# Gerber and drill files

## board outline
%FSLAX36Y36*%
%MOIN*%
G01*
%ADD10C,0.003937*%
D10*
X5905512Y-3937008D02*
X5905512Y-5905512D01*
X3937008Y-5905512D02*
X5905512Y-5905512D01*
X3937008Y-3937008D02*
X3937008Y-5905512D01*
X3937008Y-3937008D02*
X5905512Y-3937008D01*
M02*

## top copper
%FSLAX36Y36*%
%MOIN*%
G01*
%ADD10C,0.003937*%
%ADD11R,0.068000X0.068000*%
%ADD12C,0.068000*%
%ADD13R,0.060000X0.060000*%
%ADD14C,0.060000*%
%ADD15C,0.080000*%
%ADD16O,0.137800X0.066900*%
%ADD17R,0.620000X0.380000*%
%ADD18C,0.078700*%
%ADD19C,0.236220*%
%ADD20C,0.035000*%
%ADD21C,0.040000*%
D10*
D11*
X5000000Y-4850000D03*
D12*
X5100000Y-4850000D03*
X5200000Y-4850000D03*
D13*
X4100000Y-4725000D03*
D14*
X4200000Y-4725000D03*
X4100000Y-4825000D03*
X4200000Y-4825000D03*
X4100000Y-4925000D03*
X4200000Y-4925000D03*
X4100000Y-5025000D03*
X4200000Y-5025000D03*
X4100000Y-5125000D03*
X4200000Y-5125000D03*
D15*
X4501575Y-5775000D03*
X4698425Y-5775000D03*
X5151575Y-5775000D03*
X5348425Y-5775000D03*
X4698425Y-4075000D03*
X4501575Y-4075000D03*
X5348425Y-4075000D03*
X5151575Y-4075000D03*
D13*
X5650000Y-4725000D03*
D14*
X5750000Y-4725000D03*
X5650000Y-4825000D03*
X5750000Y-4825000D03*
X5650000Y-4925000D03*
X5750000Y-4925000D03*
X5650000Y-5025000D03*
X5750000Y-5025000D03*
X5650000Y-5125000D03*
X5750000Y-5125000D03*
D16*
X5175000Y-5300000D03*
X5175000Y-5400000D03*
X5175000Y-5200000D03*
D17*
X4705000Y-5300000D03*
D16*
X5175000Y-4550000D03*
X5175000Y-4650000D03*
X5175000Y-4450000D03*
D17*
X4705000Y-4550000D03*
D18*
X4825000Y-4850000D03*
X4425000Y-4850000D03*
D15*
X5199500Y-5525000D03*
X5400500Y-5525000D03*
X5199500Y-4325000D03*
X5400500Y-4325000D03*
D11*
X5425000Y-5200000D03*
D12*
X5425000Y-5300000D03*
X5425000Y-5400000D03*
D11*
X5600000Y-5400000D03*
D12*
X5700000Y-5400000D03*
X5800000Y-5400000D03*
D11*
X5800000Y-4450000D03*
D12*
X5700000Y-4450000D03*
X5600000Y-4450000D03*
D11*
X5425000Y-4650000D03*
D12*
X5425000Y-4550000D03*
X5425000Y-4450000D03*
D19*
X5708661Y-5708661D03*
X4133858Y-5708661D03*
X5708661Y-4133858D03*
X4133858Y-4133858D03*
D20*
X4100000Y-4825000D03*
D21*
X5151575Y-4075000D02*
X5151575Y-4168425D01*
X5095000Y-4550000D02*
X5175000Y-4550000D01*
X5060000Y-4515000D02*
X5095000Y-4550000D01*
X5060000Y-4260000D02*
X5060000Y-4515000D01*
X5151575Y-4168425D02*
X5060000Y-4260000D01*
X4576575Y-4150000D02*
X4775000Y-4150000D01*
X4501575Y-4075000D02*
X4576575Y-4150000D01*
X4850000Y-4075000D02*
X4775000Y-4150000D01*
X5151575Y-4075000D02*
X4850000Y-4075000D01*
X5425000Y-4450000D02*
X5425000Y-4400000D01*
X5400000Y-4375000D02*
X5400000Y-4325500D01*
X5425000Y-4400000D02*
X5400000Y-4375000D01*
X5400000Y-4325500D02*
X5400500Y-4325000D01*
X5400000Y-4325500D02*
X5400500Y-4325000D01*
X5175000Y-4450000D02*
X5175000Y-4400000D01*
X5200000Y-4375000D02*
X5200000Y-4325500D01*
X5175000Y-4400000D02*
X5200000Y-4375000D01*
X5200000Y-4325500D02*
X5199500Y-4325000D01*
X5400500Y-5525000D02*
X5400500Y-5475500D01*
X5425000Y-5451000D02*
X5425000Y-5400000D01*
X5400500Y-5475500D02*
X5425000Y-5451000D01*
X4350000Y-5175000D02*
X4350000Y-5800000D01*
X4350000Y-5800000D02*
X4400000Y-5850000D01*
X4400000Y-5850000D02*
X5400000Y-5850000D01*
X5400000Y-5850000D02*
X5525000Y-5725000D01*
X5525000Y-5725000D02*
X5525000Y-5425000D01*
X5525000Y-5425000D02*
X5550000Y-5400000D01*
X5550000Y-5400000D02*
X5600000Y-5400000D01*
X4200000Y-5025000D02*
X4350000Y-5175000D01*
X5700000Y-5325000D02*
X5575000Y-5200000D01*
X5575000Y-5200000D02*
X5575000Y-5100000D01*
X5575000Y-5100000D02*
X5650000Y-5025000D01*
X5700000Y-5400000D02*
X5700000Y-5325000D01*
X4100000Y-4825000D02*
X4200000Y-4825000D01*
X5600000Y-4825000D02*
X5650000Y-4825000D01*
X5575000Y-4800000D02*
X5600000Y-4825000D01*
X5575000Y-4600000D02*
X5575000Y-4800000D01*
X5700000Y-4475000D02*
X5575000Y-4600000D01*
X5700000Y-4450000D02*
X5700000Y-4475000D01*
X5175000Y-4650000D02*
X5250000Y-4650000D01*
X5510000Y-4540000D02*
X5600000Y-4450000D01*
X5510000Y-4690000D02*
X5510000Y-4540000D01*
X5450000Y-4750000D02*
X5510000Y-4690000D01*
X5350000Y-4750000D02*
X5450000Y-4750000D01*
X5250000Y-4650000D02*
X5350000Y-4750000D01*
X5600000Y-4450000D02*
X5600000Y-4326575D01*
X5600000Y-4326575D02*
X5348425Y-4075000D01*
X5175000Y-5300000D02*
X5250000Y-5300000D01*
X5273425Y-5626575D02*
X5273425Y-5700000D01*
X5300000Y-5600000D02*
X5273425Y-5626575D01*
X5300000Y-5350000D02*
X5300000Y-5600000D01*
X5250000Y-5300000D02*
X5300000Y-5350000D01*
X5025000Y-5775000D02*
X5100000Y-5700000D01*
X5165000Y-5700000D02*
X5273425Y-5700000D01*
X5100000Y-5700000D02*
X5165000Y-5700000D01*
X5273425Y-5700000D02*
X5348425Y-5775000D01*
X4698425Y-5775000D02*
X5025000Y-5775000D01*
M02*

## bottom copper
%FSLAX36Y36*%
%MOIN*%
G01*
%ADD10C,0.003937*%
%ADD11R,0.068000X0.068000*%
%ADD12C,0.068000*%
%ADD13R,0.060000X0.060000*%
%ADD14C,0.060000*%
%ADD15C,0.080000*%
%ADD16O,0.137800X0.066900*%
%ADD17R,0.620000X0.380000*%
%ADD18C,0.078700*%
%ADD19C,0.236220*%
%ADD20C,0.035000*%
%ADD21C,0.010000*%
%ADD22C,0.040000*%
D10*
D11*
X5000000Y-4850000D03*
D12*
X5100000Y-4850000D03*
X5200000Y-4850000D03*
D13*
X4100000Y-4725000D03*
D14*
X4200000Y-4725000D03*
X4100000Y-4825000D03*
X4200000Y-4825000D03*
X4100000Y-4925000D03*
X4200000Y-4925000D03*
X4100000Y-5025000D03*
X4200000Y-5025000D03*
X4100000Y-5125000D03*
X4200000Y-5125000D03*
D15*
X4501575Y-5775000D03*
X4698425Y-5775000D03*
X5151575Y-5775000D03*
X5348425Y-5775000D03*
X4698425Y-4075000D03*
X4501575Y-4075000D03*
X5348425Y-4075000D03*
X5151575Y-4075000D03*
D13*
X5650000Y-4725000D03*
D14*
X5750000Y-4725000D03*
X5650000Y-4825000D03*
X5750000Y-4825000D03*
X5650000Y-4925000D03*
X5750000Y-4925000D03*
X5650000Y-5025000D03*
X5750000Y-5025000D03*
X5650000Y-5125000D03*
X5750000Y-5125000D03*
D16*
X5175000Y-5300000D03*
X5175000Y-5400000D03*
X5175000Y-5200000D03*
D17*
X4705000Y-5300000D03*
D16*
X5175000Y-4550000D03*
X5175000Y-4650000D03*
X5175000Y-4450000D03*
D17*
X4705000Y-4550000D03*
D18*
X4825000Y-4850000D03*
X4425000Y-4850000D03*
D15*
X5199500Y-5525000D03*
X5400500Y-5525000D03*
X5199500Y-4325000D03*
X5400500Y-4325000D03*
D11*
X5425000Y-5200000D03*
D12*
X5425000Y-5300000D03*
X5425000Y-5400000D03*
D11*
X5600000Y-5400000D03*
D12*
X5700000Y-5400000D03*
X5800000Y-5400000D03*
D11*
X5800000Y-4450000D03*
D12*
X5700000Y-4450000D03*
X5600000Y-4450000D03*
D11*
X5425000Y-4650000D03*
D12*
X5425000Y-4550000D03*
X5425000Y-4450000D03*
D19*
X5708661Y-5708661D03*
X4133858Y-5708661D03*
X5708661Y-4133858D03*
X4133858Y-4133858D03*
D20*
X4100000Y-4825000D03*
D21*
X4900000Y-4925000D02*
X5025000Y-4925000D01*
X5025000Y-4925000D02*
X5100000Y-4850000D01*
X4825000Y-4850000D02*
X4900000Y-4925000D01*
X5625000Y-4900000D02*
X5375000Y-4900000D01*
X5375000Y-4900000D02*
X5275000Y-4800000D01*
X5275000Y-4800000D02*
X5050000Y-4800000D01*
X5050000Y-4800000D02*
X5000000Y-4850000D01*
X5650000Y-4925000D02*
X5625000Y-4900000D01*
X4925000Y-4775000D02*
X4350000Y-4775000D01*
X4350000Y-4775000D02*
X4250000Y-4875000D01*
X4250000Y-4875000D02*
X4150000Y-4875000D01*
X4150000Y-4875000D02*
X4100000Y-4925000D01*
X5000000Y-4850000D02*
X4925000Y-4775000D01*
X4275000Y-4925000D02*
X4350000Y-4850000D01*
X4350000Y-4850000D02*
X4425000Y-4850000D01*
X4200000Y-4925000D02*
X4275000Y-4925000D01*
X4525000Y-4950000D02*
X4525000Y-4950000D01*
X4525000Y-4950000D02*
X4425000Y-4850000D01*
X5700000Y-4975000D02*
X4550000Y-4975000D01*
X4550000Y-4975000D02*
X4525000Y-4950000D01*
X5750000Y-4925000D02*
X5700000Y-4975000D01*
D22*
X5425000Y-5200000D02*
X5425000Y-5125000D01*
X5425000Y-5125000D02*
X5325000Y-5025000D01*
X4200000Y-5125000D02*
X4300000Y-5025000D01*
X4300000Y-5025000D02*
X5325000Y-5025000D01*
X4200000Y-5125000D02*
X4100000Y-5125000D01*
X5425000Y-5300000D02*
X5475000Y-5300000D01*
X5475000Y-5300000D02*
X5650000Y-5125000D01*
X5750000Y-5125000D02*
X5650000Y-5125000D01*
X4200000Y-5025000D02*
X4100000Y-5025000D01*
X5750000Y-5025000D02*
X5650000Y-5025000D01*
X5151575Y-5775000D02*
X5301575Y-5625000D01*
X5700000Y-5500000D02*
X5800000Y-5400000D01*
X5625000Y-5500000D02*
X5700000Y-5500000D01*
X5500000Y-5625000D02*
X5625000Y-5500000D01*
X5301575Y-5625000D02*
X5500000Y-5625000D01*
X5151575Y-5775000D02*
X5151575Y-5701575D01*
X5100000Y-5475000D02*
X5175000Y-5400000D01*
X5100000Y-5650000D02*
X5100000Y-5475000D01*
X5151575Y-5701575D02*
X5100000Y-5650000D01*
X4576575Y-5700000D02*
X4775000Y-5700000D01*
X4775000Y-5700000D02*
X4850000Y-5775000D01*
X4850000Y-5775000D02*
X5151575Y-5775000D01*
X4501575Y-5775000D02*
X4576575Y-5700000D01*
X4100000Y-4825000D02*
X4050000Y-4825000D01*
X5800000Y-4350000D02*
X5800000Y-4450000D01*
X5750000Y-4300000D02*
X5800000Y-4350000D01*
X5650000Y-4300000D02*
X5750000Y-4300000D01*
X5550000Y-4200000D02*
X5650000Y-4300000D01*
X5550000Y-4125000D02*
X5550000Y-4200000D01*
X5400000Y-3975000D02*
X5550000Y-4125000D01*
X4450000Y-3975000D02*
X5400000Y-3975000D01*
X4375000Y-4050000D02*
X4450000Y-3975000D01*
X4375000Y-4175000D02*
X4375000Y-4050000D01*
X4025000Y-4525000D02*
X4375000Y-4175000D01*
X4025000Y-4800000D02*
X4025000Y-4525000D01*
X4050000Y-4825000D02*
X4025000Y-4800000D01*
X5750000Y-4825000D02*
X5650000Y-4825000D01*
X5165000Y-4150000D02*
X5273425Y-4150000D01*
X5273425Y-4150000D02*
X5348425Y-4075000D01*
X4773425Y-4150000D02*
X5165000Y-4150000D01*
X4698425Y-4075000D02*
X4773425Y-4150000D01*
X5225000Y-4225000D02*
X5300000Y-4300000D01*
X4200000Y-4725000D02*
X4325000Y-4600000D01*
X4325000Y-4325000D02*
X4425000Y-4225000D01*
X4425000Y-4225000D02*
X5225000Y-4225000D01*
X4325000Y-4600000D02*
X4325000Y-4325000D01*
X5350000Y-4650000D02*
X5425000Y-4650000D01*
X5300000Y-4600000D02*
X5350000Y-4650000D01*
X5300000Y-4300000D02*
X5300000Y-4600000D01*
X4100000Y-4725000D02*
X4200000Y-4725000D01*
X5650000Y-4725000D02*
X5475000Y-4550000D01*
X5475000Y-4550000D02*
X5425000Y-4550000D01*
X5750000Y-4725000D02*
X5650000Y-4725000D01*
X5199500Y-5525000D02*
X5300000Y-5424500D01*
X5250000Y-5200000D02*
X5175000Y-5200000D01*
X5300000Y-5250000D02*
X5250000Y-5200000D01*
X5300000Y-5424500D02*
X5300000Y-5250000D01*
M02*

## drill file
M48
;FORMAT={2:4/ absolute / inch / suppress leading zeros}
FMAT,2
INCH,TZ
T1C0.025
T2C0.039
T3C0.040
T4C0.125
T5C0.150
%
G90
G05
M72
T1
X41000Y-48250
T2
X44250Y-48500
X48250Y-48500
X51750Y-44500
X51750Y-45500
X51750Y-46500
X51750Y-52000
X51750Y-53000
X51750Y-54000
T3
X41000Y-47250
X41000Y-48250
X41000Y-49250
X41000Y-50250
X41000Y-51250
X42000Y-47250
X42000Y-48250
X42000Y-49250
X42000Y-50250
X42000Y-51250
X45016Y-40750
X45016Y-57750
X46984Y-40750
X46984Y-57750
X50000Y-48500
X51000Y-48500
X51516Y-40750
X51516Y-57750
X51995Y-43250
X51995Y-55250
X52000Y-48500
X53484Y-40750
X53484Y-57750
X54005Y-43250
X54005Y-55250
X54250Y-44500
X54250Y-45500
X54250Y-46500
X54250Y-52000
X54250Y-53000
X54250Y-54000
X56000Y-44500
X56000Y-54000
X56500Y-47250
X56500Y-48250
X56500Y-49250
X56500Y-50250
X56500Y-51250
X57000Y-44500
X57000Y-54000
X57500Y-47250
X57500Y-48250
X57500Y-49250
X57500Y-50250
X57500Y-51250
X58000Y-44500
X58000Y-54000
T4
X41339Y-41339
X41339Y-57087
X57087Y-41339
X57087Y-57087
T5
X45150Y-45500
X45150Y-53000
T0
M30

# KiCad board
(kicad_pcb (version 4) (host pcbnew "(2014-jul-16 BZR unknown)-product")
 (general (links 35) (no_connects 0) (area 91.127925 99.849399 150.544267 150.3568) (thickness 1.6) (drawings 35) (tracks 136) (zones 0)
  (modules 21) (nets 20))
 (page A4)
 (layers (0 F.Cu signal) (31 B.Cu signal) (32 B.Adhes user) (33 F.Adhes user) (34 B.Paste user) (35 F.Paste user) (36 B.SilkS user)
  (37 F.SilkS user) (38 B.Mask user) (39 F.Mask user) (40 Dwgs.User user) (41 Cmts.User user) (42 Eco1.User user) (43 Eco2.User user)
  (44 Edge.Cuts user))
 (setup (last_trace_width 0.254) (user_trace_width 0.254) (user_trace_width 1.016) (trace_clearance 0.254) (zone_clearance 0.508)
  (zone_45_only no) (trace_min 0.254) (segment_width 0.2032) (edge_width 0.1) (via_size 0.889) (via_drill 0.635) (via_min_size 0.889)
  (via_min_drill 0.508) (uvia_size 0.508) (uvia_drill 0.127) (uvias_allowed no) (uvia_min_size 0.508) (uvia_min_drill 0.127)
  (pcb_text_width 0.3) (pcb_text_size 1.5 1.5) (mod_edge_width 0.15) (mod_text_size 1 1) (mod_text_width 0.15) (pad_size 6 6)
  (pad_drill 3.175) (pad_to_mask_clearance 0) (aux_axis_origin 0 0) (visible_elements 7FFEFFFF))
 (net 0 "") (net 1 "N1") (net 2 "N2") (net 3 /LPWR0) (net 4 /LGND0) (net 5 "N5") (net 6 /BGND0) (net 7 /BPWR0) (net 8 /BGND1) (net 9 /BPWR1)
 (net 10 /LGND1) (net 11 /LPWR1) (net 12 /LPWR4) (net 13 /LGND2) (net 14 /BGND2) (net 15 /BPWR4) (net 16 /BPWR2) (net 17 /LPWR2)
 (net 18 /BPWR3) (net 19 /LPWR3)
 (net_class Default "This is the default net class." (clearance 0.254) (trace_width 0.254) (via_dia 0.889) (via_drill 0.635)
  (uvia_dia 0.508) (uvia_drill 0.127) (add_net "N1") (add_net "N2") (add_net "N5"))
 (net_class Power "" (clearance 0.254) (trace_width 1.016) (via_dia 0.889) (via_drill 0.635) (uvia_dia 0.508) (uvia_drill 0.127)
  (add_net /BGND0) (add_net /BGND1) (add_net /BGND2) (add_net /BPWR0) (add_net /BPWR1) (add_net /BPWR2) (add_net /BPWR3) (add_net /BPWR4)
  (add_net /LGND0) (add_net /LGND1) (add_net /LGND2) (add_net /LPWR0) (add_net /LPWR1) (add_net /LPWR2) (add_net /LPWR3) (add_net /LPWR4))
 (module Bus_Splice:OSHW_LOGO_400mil (layer B.Cu) (at 124.333 113.03 180)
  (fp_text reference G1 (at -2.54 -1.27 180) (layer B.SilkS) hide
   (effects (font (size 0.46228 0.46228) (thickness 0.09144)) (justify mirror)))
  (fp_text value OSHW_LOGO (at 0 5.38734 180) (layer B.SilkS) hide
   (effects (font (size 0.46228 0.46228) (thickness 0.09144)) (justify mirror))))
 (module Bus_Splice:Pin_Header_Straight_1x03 (layer F.Cu) (at 129.54 123.19)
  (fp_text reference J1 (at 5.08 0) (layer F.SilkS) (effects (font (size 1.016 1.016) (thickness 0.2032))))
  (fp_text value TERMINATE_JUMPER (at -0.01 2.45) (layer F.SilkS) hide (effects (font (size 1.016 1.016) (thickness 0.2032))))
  (pad 1 thru_hole rect (at -2.54 0) (size 1.7272 1.7272) (drill 1.016) (layers *.Cu *.Mask F.SilkS) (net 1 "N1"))
  (pad 2 thru_hole circle (at 0 0) (size 1.7272 1.7272) (drill 1.016) (layers *.Cu *.Mask F.SilkS) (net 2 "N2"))
  (pad 3 thru_hole circle (at 2.54 0) (size 1.7272 1.7272) (drill 1.016) (layers *.Cu *.Mask F.SilkS)))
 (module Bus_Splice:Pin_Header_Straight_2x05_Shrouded (layer F.Cu) (at 105.41 125.095 270)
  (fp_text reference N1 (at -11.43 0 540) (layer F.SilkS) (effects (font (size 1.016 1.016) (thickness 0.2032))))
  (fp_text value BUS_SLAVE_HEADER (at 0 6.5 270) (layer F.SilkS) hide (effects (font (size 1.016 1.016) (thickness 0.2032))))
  (pad 1 thru_hole rect (at -5.08 1.27 270) (size 1.524 1.524) (drill 1.016) (layers *.Cu *.Mask F.SilkS) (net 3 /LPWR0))
  (pad 2 thru_hole circle (at -5.08 -1.27 270) (size 1.524 1.524) (drill 1.016) (layers *.Cu *.Mask F.SilkS) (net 3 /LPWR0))
  (pad 3 thru_hole circle (at -2.54 1.27 270) (size 1.524 1.524) (drill 1.016) (layers *.Cu *.Mask F.SilkS) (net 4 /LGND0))
  (pad 4 thru_hole circle (at -2.54 -1.27 270) (size 1.524 1.524) (drill 1.016) (layers *.Cu *.Mask F.SilkS) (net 4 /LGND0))
  (pad 5 thru_hole circle (at 0 1.27 270) (size 1.524 1.524) (drill 1.016) (layers *.Cu *.Mask F.SilkS) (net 1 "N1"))
  (pad 6 thru_hole circle (at 0 -1.27 270) (size 1.524 1.524) (drill 1.016) (layers *.Cu *.Mask F.SilkS) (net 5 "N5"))
  (pad 7 thru_hole circle (at 2.54 1.27 270) (size 1.524 1.524) (drill 1.016) (layers *.Cu *.Mask F.SilkS) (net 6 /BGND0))
  (pad 8 thru_hole circle (at 2.54 -1.27 270) (size 1.524 1.524) (drill 1.016) (layers *.Cu *.Mask F.SilkS) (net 6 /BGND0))
  (pad 9 thru_hole circle (at 5.08 1.27 270) (size 1.524 1.524) (drill 1.016) (layers *.Cu *.Mask F.SilkS) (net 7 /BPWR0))
  (pad 10 thru_hole circle (at 5.08 -1.27 270) (size 1.524 1.524) (drill 1.016) (layers *.Cu *.Mask F.SilkS) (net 7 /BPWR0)))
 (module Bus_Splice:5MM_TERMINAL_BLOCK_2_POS (layer F.Cu) (at 116.84 146.685)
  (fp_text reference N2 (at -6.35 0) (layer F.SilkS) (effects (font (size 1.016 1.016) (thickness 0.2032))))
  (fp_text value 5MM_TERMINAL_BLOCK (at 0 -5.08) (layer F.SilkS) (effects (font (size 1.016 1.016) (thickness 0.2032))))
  (pad 1 thru_hole circle (at -2.5 0) (size 2.032 2.032) (drill 1.016) (layers *.Cu *.Mask) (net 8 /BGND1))
  (pad 2 thru_hole circle (at 2.5 0) (size 2.032 2.032) (drill 1.016) (layers *.Cu *.Mask) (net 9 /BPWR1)))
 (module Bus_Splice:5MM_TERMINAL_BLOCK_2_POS (layer F.Cu) (at 133.35 146.685)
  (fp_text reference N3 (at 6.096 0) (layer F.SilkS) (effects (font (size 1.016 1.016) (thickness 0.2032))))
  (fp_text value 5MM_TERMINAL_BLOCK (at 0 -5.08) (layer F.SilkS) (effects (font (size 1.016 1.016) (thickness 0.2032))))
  (pad 1 thru_hole circle (at -2.5 0) (size 2.032 2.032) (drill 1.016) (layers *.Cu *.Mask) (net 8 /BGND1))
  (pad 2 thru_hole circle (at 2.5 0) (size 2.032 2.032) (drill 1.016) (layers *.Cu *.Mask) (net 9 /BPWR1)))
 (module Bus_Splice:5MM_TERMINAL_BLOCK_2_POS (layer F.Cu) (at 116.84 103.505 180)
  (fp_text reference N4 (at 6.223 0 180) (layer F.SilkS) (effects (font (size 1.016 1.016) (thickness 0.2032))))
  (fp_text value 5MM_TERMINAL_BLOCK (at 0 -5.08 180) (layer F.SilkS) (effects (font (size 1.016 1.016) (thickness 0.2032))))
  (pad 1 thru_hole circle (at -2.5 0 180) (size 2.032 2.032) (drill 1.016) (layers *.Cu *.Mask) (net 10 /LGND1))
  (pad 2 thru_hole circle (at 2.5 0 180) (size 2.032 2.032) (drill 1.016) (layers *.Cu *.Mask) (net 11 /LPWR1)))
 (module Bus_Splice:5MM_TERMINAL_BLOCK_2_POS (layer F.Cu) (at 133.35 103.505 180)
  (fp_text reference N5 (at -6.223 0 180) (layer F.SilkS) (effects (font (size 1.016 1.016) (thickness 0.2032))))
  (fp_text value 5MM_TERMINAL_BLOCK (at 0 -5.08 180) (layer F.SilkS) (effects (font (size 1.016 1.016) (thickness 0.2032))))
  (pad 1 thru_hole circle (at -2.5 0 180) (size 2.032 2.032) (drill 1.016) (layers *.Cu *.Mask) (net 10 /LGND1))
  (pad 2 thru_hole circle (at 2.5 0 180) (size 2.032 2.032) (drill 1.016) (layers *.Cu *.Mask) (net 11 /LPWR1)))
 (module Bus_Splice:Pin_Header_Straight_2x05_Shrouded (layer F.Cu) (at 144.78 125.095 270)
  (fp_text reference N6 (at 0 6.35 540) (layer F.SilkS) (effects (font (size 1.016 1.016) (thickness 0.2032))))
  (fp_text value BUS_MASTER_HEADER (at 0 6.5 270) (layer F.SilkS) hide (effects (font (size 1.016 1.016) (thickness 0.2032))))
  (pad 1 thru_hole rect (at -5.08 1.27 270) (size 1.524 1.524) (drill 1.016) (layers *.Cu *.Mask F.SilkS) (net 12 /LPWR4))
  (pad 2 thru_hole circle (at -5.08 -1.27 270) (size 1.524 1.524) (drill 1.016) (layers *.Cu *.Mask F.SilkS) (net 12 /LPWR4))
  (pad 3 thru_hole circle (at -2.54 1.27 270) (size 1.524 1.524) (drill 1.016) (layers *.Cu *.Mask F.SilkS) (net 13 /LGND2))
  (pad 4 thru_hole circle (at -2.54 -1.27 270) (size 1.524 1.524) (drill 1.016) (layers *.Cu *.Mask F.SilkS) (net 13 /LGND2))
  (pad 5 thru_hole circle (at 0 1.27 270) (size 1.524 1.524) (drill 1.016) (layers *.Cu *.Mask F.SilkS) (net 1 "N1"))
  (pad 6 thru_hole circle (at 0 -1.27 270) (size 1.524 1.524) (drill 1.016) (layers *.Cu *.Mask F.SilkS) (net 5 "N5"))
  (pad 7 thru_hole circle (at 2.54 1.27 270) (size 1.524 1.524) (drill 1.016) (layers *.Cu *.Mask F.SilkS) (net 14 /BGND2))
  (pad 8 thru_hole circle (at 2.54 -1.27 270) (size 1.524 1.524) (drill 1.016) (layers *.Cu *.Mask F.SilkS) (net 14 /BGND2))
  (pad 9 thru_hole circle (at 5.08 1.27 270) (size 1.524 1.524) (drill 1.016) (layers *.Cu *.Mask F.SilkS) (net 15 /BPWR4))
  (pad 10 thru_hole circle (at 5.08 -1.27 270) (size 1.524 1.524) (drill 1.016) (layers *.Cu *.Mask F.SilkS) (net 15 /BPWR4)))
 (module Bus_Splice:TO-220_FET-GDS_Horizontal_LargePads (layer F.Cu) (at 131.445 134.62 90)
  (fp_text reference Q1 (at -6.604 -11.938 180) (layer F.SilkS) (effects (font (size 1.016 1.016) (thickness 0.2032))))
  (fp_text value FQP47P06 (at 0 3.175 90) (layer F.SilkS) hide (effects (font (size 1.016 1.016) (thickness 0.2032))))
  (pad D thru_hole oval (at 0 0 180) (size 3.50012 1.69926) (drill 1.00076) (layers *.Cu *.Mask F.SilkS) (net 9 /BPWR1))
  (pad G thru_hole oval (at -2.54 0 180) (size 3.50012 1.69926) (drill 1.00076) (layers *.Cu *.Mask F.SilkS) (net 8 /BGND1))
  (pad S thru_hole oval (at 2.54 0 180) (size 3.50012 1.69926) (drill 1.00076) (layers *.Cu *.Mask F.SilkS) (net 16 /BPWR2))
  (pad 2 thru_hole rect (at 0 -16.764 180) (size 15.748 9.652) (drill 3.79984 (offset -4.826 0)) (layers *.Cu F.SilkS F.Mask)))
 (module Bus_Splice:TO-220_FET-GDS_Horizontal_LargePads (layer F.Cu) (at 131.445 115.57 90)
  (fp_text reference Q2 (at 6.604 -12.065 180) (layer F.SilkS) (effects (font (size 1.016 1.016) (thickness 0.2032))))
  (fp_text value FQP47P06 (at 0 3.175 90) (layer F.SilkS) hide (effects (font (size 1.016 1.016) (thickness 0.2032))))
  (pad D thru_hole oval (at 0 0 180) (size 3.50012 1.69926) (drill 1.00076) (layers *.Cu *.Mask F.SilkS) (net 11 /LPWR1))
  (pad G thru_hole oval (at -2.54 0 180) (size 3.50012 1.69926) (drill 1.00076) (layers *.Cu *.Mask F.SilkS) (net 10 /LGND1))
  (pad S thru_hole oval (at 2.54 0 180) (size 3.50012 1.69926) (drill 1.00076) (layers *.Cu *.Mask F.SilkS) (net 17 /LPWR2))
  (pad 2 thru_hole rect (at 0 -16.764 180) (size 15.748 9.652) (drill 3.79984 (offset -4.826 0)) (layers *.Cu F.SilkS F.Mask)))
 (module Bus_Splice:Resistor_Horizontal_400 (layer F.Cu) (at 117.475 123.19 180)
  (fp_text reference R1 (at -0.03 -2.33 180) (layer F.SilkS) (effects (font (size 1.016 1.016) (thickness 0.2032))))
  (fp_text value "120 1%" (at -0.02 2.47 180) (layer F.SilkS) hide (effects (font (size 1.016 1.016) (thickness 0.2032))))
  (pad 1 thru_hole circle (at -5.08 0 180) (size 1.99898 1.99898) (drill 1.00076) (layers *.Cu *.SilkS *.Mask) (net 2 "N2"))
  (pad 2 thru_hole circle (at 5.08 0 180) (size 1.99898 1.99898) (drill 1.00076) (layers *.Cu *.SilkS *.Mask) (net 5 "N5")))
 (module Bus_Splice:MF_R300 (layer F.Cu) (at 134.62 140.335)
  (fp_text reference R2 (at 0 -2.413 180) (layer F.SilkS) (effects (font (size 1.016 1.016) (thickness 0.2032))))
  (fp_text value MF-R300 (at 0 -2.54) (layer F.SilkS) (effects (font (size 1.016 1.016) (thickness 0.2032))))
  (pad 1 thru_hole circle (at -2.5527 0) (size 2.032 2.032) (drill 1.016) (layers *.Cu *.Mask) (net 16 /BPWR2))
  (pad 2 thru_hole circle (at 2.5527 0) (size 2.032 2.032) (drill 1.016) (layers *.Cu *.Mask) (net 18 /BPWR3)))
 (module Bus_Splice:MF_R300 (layer F.Cu) (at 134.62 109.855)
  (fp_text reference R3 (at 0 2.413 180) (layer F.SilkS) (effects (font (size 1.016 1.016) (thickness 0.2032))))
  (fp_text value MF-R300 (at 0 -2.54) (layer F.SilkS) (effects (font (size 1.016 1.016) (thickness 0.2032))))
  (pad 1 thru_hole circle (at -2.5527 0) (size 2.032 2.032) (drill 1.016) (layers *.Cu *.Mask) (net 17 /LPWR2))
  (pad 2 thru_hole circle (at 2.5527 0) (size 2.032 2.032) (drill 1.016) (layers *.Cu *.Mask) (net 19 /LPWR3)))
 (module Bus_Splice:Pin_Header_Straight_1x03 (layer F.Cu) (at 137.795 134.62 270)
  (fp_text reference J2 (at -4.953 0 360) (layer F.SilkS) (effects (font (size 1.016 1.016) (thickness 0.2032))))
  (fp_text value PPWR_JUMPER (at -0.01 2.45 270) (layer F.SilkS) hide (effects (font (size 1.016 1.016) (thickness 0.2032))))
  (pad 1 thru_hole rect (at -2.54 0 270) (size 1.7272 1.7272) (drill 1.016) (layers *.Cu *.Mask F.SilkS) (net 7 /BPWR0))
  (pad 2 thru_hole circle (at 0 0 270) (size 1.7272 1.7272) (drill 1.016) (layers *.Cu *.Mask F.SilkS) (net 15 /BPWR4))
  (pad 3 thru_hole circle (at 2.54 0 270) (size 1.7272 1.7272) (drill 1.016) (layers *.Cu *.Mask F.SilkS) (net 18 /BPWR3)))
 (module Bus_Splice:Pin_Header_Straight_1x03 (layer F.Cu) (at 144.78 137.16)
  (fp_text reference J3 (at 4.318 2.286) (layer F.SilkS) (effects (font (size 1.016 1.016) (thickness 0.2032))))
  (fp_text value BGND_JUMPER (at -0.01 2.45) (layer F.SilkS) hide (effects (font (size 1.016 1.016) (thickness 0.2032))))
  (pad 1 thru_hole rect (at -2.54 0) (size 1.7272 1.7272) (drill 1.016) (layers *.Cu *.Mask F.SilkS) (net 6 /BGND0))
  (pad 2 thru_hole circle (at 0 0) (size 1.7272 1.7272) (drill 1.016) (layers *.Cu *.Mask F.SilkS) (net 14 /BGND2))
  (pad 3 thru_hole circle (at 2.54 0) (size 1.7272 1.7272) (drill 1.016) (layers *.Cu *.Mask F.SilkS) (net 8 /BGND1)))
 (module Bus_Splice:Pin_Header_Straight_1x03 (layer F.Cu) (at 144.78 113.03 180)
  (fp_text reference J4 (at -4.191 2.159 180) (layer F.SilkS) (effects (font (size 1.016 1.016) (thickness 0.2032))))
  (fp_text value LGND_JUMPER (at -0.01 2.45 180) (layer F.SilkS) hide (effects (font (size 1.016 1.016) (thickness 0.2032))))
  (pad 1 thru_hole rect (at -2.54 0 180) (size 1.7272 1.7272) (drill 1.016) (layers *.Cu *.Mask F.SilkS) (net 4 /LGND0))
  (pad 2 thru_hole circle (at 0 0 180) (size 1.7272 1.7272) (drill 1.016) (layers *.Cu *.Mask F.SilkS) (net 13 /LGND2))
  (pad 3 thru_hole circle (at 2.54 0 180) (size 1.7272 1.7272) (drill 1.016) (layers *.Cu *.Mask F.SilkS) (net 10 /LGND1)))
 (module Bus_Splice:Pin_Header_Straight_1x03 (layer F.Cu) (at 137.795 115.57 90)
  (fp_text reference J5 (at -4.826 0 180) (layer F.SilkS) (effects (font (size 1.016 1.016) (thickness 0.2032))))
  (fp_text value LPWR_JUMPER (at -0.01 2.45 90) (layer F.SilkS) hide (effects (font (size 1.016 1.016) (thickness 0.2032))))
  (pad 1 thru_hole rect (at -2.54 0 90) (size 1.7272 1.7272) (drill 1.016) (layers *.Cu *.Mask F.SilkS) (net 3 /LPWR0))
  (pad 2 thru_hole circle (at 0 0 90) (size 1.7272 1.7272) (drill 1.016) (layers *.Cu *.Mask F.SilkS) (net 12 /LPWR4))
  (pad 3 thru_hole circle (at 2.54 0 90) (size 1.7272 1.7272) (drill 1.016) (layers *.Cu *.Mask F.SilkS) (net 19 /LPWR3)))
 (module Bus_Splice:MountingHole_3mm (layer F.Cu) (at 145 145)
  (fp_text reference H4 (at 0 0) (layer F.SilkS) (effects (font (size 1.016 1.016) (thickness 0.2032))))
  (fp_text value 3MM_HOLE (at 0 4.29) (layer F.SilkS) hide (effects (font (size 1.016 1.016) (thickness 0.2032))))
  (pad 1 thru_hole circle (at 0 0) (size 6 6) (drill 3.175) (layers *.Cu)))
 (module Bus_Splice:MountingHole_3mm (layer F.Cu) (at 105 145)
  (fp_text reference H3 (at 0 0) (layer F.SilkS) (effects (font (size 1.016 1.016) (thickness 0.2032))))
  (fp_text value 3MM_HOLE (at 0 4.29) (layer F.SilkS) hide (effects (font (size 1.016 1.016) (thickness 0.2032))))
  (pad 1 thru_hole circle (at 0 0) (size 6 6) (drill 3.175) (layers *.Cu)))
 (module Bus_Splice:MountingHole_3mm (layer F.Cu) (at 145 105)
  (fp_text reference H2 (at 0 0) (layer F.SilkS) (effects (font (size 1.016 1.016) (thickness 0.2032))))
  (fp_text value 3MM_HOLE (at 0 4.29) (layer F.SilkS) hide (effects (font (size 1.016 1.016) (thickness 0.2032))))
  (pad 1 thru_hole circle (at 0 0) (size 6 6) (drill 3.175) (layers *.Cu)))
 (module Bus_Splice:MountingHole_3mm (layer F.Cu) (at 105 105)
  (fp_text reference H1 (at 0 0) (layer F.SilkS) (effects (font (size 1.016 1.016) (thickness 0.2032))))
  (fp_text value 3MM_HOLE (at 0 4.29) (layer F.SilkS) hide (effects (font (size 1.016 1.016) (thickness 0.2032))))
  (pad 1 thru_hole circle (at 0 0) (size 6 6) (drill 3.175) (layers *.Cu)))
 (gr_line (start 150 100) (end 150 150) (angle 90) (layer Edge.Cuts) (width 0.1))
 (gr_line (start 100 150) (end 150 150) (angle 90) (layer Edge.Cuts) (width 0.1))
 (gr_line (start 100 100) (end 100 150) (angle 90) (layer Edge.Cuts) (width 0.1))
 (gr_line (start 100 100) (end 150 100) (angle 90) (layer Edge.Cuts) (width 0.1))
 (segment (start 130.85 103.505) (end 130.85 105.878) (width 1.016) (layer F.Cu) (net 11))
 (segment (start 129.413 115.57) (end 131.445 115.57) (width 1.016) (layer F.Cu) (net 11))
 (segment (start 128.524 114.681) (end 129.413 115.57) (width 1.016) (layer F.Cu) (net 11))
 (segment (start 128.524 108.204) (end 128.524 114.681) (width 1.016) (layer F.Cu) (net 11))
 (segment (start 130.85 105.878) (end 128.524 108.204) (width 1.016) (layer F.Cu) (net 11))
 (segment (start 116.245 105.41) (end 121.285 105.41) (width 1.016) (layer F.Cu) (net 11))
 (segment (start 114.34 103.505) (end 116.245 105.41) (width 1.016) (layer F.Cu) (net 11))
 (segment (start 123.19 103.505) (end 121.285 105.41) (width 1.016) (layer F.Cu) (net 11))
 (segment (start 130.85 103.505) (end 123.19 103.505) (width 1.016) (layer F.Cu) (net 11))
 (segment (start 137.795 113.03) (end 137.795 111.76) (width 1.016) (layer F.Cu) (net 19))
 (segment (start 137.16 111.125) (end 137.16 109.8677) (width 1.016) (layer F.Cu) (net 19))
 (segment (start 137.795 111.76) (end 137.16 111.125) (width 1.016) (layer F.Cu) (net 19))
 (segment (start 137.16 109.8677) (end 137.1727 109.855) (width 1.016) (layer F.Cu) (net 19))
 (segment (start 137.16 109.8677) (end 137.1727 109.855) (width 1.016) (layer F.Cu) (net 19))
 (segment (start 131.445 113.03) (end 131.445 111.76) (width 1.016) (layer F.Cu) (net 17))
 (segment (start 132.08 111.125) (end 132.08 109.8677) (width 1.016) (layer F.Cu) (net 17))
 (segment (start 131.445 111.76) (end 132.08 111.125) (width 1.016) (layer F.Cu) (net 17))
 (segment (start 132.08 109.8677) (end 132.0673 109.855) (width 1.016) (layer F.Cu) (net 17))
 (segment (start 124.46 125.095) (end 127.635 125.095) (width 0.254) (layer B.Cu) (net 2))
 (segment (start 127.635 125.095) (end 129.54 123.19) (width 0.254) (layer B.Cu) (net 2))
 (segment (start 122.555 123.19) (end 124.46 125.095) (width 0.254) (layer B.Cu) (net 2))
 (segment (start 142.875 124.46) (end 136.525 124.46) (width 0.254) (layer B.Cu) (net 1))
 (segment (start 136.525 124.46) (end 133.985 121.92) (width 0.254) (layer B.Cu) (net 1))
 (segment (start 133.985 121.92) (end 128.27 121.92) (width 0.254) (layer B.Cu) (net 1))
 (segment (start 128.27 121.92) (end 127 123.19) (width 0.254) (layer B.Cu) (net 1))
 (segment (start 143.51 125.095) (end 142.875 124.46) (width 0.254) (layer B.Cu) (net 1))
 (segment (start 125.095 121.285) (end 110.49 121.285) (width 0.254) (layer B.Cu) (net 1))
 (segment (start 110.49 121.285) (end 107.95 123.825) (width 0.254) (layer B.Cu) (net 1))
 (segment (start 107.95 123.825) (end 105.41 123.825) (width 0.254) (layer B.Cu) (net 1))
 (segment (start 105.41 123.825) (end 104.14 125.095) (width 0.254) (layer B.Cu) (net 1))
 (segment (start 127 123.19) (end 125.095 121.285) (width 0.254) (layer B.Cu) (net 1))
 (segment (start 108.585 125.095) (end 110.49 123.19) (width 0.254) (layer B.Cu) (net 5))
 (segment (start 110.49 123.19) (end 112.395 123.19) (width 0.254) (layer B.Cu) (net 5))
 (segment (start 106.68 125.095) (end 108.585 125.095) (width 0.254) (layer B.Cu) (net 5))
 (segment (start 114.935 125.73) (end 114.935 125.73) (width 0.254) (layer B.Cu) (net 5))
 (segment (start 114.935 125.73) (end 112.395 123.19) (width 0.254) (layer B.Cu) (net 5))
 (segment (start 144.78 126.365) (end 115.57 126.365) (width 0.254) (layer B.Cu) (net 5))
 (segment (start 115.57 126.365) (end 114.935 125.73) (width 0.254) (layer B.Cu) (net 5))
 (segment (start 146.05 125.095) (end 144.78 126.365) (width 0.254) (layer B.Cu) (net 5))
 (segment (start 137.795 132.08) (end 137.795 130.175) (width 1.016) (layer B.Cu) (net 7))
 (segment (start 137.795 130.175) (end 135.255 127.635) (width 1.016) (layer B.Cu) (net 7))
 (segment (start 106.68 130.175) (end 109.22 127.635) (width 1.016) (layer B.Cu) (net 7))
 (segment (start 109.22 127.635) (end 135.255 127.635) (width 1.016) (layer B.Cu) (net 7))
 (segment (start 106.68 130.175) (end 104.14 130.175) (width 1.016) (layer B.Cu) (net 7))
 (segment (start 137.795 134.62) (end 139.065 134.62) (width 1.016) (layer B.Cu) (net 15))
 (segment (start 139.065 134.62) (end 143.51 130.175) (width 1.016) (layer B.Cu) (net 15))
 (segment (start 146.05 130.175) (end 143.51 130.175) (width 1.016) (layer B.Cu) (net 15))
 (segment (start 137.1727 140.335) (end 137.1727 139.0777) (width 1.016) (layer F.Cu) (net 18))
 (segment (start 137.795 138.4554) (end 137.795 137.16) (width 1.016) (layer F.Cu) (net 18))
 (segment (start 137.1727 139.0777) (end 137.795 138.4554) (width 1.016) (layer F.Cu) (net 18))
 (segment (start 106.68 127.635) (end 104.14 127.635) (width 1.016) (layer B.Cu) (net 6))
 (segment (start 110.49 131.445) (end 110.49 147.32) (width 1.016) (layer F.Cu) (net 6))
 (segment (start 110.49 147.32) (end 111.76 148.59) (width 1.016) (layer F.Cu) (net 6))
 (segment (start 111.76 148.59) (end 137.16 148.59) (width 1.016) (layer F.Cu) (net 6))
 (segment (start 137.16 148.59) (end 140.335 145.415) (width 1.016) (layer F.Cu) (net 6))
 (segment (start 140.335 145.415) (end 140.335 137.795) (width 1.016) (layer F.Cu) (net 6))
 (segment (start 140.335 137.795) (end 140.97 137.16) (width 1.016) (layer F.Cu) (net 6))
 (segment (start 140.97 137.16) (end 142.24 137.16) (width 1.016) (layer F.Cu) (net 6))
 (segment (start 106.68 127.635) (end 110.49 131.445) (width 1.016) (layer F.Cu) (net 6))
 (segment (start 146.05 127.635) (end 143.51 127.635) (width 1.016) (layer B.Cu) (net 14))
 (segment (start 144.78 135.255) (end 141.605 132.08) (width 1.016) (layer F.Cu) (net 14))
 (segment (start 141.605 132.08) (end 141.605 129.54) (width 1.016) (layer F.Cu) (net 14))
 (segment (start 141.605 129.54) (end 143.51 127.635) (width 1.016) (layer F.Cu) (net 14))
 (segment (start 144.78 137.16) (end 144.78 135.255) (width 1.016) (layer F.Cu) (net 14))
 (segment (start 130.85 146.685) (end 134.66 142.875) (width 1.016) (layer B.Cu) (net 8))
 (segment (start 144.78 139.7) (end 147.32 137.16) (width 1.016) (layer B.Cu) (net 8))
 (segment (start 142.875 139.7) (end 144.78 139.7) (width 1.016) (layer B.Cu) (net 8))
 (segment (start 139.7 142.875) (end 142.875 139.7) (width 1.016) (layer B.Cu) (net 8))
 (segment (start 134.66 142.875) (end 139.7 142.875) (width 1.016) (layer B.Cu) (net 8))
 (segment (start 130.85 146.685) (end 130.85 144.82) (width 1.016) (layer B.Cu) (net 8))
 (segment (start 129.54 139.065) (end 131.445 137.16) (width 1.016) (layer B.Cu) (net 8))
 (segment (start 129.54 143.51) (end 129.54 139.065) (width 1.016) (layer B.Cu) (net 8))
 (segment (start 130.85 144.82) (end 129.54 143.51) (width 1.016) (layer B.Cu) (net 8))
 (segment (start 116.245 144.78) (end 121.285 144.78) (width 1.016) (layer B.Cu) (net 8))
 (segment (start 121.285 144.78) (end 123.19 146.685) (width 1.016) (layer B.Cu) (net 8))
 (segment (start 123.19 146.685) (end 130.85 146.685) (width 1.016) (layer B.Cu) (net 8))
 (segment (start 114.34 146.685) (end 116.245 144.78) (width 1.016) (layer B.Cu) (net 8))
 (segment (start 104.14 122.555) (end 102.87 122.555) (width 1.016) (layer B.Cu) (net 4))
 (segment (start 147.32 110.49) (end 147.32 113.03) (width 1.016) (layer B.Cu) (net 4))
 (segment (start 146.05 109.22) (end 147.32 110.49) (width 1.016) (layer B.Cu) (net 4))
 (segment (start 143.51 109.22) (end 146.05 109.22) (width 1.016) (layer B.Cu) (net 4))
 (segment (start 140.97 106.68) (end 143.51 109.22) (width 1.016) (layer B.Cu) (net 4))
 (segment (start 140.97 104.775) (end 140.97 106.68) (width 1.016) (layer B.Cu) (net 4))
 (segment (start 137.16 100.965) (end 140.97 104.775) (width 1.016) (layer B.Cu) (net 4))
 (segment (start 113.03 100.965) (end 137.16 100.965) (width 1.016) (layer B.Cu) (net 4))
 (segment (start 111.125 102.87) (end 113.03 100.965) (width 1.016) (layer B.Cu) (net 4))
 (segment (start 111.125 106.045) (end 111.125 102.87) (width 1.016) (layer B.Cu) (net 4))
 (segment (start 102.235 114.935) (end 111.125 106.045) (width 1.016) (layer B.Cu) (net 4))
 (segment (start 102.235 121.92) (end 102.235 114.935) (width 1.016) (layer B.Cu) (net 4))
 (segment (start 102.87 122.555) (end 102.235 121.92) (width 1.016) (layer B.Cu) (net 4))
 (segment (start 104.14 122.555) (end 106.68 122.555) (width 1.016) (layer F.Cu) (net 4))
 (via (at 104.14 122.555) (size 0.889) (layers F.Cu B.Cu) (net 4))
 (segment (start 146.05 122.555) (end 143.51 122.555) (width 1.016) (layer B.Cu) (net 13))
 (segment (start 142.24 122.555) (end 143.51 122.555) (width 1.016) (layer F.Cu) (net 13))
 (segment (start 141.605 121.92) (end 142.24 122.555) (width 1.016) (layer F.Cu) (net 13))
 (segment (start 141.605 116.84) (end 141.605 121.92) (width 1.016) (layer F.Cu) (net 13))
 (segment (start 144.78 113.665) (end 141.605 116.84) (width 1.016) (layer F.Cu) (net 13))
 (segment (start 144.78 113.03) (end 144.78 113.665) (width 1.016) (layer F.Cu) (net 13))
 (segment (start 131.445 118.11) (end 133.35 118.11) (width 1.016) (layer F.Cu) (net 10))
 (segment (start 139.954 115.316) (end 142.24 113.03) (width 1.016) (layer F.Cu) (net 10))
 (segment (start 139.954 119.126) (end 139.954 115.316) (width 1.016) (layer F.Cu) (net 10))
 (segment (start 138.43 120.65) (end 139.954 119.126) (width 1.016) (layer F.Cu) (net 10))
 (segment (start 135.89 120.65) (end 138.43 120.65) (width 1.016) (layer F.Cu) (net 10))
 (segment (start 133.35 118.11) (end 135.89 120.65) (width 1.016) (layer F.Cu) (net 10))
 (segment (start 142.24 113.03) (end 142.24 109.895) (width 1.016) (layer F.Cu) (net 10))
 (segment (start 142.24 109.895) (end 135.85 103.505) (width 1.016) (layer F.Cu) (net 10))
 (segment (start 131.191 105.41) (end 133.945 105.41) (width 1.016) (layer B.Cu) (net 10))
 (segment (start 133.945 105.41) (end 135.85 103.505) (width 1.016) (layer B.Cu) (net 10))
 (segment (start 121.245 105.41) (end 131.191 105.41) (width 1.016) (layer B.Cu) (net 10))
 (segment (start 119.34 103.505) (end 121.245 105.41) (width 1.016) (layer B.Cu) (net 10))
 (segment (start 132.715 107.315) (end 134.62 109.22) (width 1.016) (layer B.Cu) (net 3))
 (segment (start 106.68 120.015) (end 109.855 116.84) (width 1.016) (layer B.Cu) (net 3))
 (segment (start 109.855 109.855) (end 112.395 107.315) (width 1.016) (layer B.Cu) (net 3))
 (segment (start 112.395 107.315) (end 132.715 107.315) (width 1.016) (layer B.Cu) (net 3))
 (segment (start 109.855 116.84) (end 109.855 109.855) (width 1.016) (layer B.Cu) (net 3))
 (segment (start 135.89 118.11) (end 137.795 118.11) (width 1.016) (layer B.Cu) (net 3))
 (segment (start 134.62 116.84) (end 135.89 118.11) (width 1.016) (layer B.Cu) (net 3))
 (segment (start 134.62 109.22) (end 134.62 116.84) (width 1.016) (layer B.Cu) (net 3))
 (segment (start 104.14 120.015) (end 106.68 120.015) (width 1.016) (layer B.Cu) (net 3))
 (segment (start 143.51 120.015) (end 139.065 115.57) (width 1.016) (layer B.Cu) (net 12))
 (segment (start 139.065 115.57) (end 137.795 115.57) (width 1.016) (layer B.Cu) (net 12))
 (segment (start 146.05 120.015) (end 143.51 120.015) (width 1.016) (layer B.Cu) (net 12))
 (segment (start 131.445 134.62) (end 133.35 134.62) (width 1.016) (layer F.Cu) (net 9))
 (segment (start 133.945 142.915) (end 133.945 144.78) (width 1.016) (layer F.Cu) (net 9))
 (segment (start 134.62 142.24) (end 133.945 142.915) (width 1.016) (layer F.Cu) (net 9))
 (segment (start 134.62 135.89) (end 134.62 142.24) (width 1.016) (layer F.Cu) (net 9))
 (segment (start 133.35 134.62) (end 134.62 135.89) (width 1.016) (layer F.Cu) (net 9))
 (segment (start 127.635 146.685) (end 129.54 144.78) (width 1.016) (layer F.Cu) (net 9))
 (segment (start 131.191 144.78) (end 133.945 144.78) (width 1.016) (layer F.Cu) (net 9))
 (segment (start 129.54 144.78) (end 131.191 144.78) (width 1.016) (layer F.Cu) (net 9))
 (segment (start 133.945 144.78) (end 135.85 146.685) (width 1.016) (layer F.Cu) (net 9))
 (segment (start 119.34 146.685) (end 127.635 146.685) (width 1.016) (layer F.Cu) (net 9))
 (segment (start 132.0673 140.335) (end 134.62 137.7823) (width 1.016) (layer B.Cu) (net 16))
 (segment (start 133.35 132.08) (end 131.445 132.08) (width 1.016) (layer B.Cu) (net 16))
 (segment (start 134.62 133.35) (end 133.35 132.08) (width 1.016) (layer B.Cu) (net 16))
 (segment (start 134.62 137.7823) (end 134.62 133.35) (width 1.016) (layer B.Cu) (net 16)))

